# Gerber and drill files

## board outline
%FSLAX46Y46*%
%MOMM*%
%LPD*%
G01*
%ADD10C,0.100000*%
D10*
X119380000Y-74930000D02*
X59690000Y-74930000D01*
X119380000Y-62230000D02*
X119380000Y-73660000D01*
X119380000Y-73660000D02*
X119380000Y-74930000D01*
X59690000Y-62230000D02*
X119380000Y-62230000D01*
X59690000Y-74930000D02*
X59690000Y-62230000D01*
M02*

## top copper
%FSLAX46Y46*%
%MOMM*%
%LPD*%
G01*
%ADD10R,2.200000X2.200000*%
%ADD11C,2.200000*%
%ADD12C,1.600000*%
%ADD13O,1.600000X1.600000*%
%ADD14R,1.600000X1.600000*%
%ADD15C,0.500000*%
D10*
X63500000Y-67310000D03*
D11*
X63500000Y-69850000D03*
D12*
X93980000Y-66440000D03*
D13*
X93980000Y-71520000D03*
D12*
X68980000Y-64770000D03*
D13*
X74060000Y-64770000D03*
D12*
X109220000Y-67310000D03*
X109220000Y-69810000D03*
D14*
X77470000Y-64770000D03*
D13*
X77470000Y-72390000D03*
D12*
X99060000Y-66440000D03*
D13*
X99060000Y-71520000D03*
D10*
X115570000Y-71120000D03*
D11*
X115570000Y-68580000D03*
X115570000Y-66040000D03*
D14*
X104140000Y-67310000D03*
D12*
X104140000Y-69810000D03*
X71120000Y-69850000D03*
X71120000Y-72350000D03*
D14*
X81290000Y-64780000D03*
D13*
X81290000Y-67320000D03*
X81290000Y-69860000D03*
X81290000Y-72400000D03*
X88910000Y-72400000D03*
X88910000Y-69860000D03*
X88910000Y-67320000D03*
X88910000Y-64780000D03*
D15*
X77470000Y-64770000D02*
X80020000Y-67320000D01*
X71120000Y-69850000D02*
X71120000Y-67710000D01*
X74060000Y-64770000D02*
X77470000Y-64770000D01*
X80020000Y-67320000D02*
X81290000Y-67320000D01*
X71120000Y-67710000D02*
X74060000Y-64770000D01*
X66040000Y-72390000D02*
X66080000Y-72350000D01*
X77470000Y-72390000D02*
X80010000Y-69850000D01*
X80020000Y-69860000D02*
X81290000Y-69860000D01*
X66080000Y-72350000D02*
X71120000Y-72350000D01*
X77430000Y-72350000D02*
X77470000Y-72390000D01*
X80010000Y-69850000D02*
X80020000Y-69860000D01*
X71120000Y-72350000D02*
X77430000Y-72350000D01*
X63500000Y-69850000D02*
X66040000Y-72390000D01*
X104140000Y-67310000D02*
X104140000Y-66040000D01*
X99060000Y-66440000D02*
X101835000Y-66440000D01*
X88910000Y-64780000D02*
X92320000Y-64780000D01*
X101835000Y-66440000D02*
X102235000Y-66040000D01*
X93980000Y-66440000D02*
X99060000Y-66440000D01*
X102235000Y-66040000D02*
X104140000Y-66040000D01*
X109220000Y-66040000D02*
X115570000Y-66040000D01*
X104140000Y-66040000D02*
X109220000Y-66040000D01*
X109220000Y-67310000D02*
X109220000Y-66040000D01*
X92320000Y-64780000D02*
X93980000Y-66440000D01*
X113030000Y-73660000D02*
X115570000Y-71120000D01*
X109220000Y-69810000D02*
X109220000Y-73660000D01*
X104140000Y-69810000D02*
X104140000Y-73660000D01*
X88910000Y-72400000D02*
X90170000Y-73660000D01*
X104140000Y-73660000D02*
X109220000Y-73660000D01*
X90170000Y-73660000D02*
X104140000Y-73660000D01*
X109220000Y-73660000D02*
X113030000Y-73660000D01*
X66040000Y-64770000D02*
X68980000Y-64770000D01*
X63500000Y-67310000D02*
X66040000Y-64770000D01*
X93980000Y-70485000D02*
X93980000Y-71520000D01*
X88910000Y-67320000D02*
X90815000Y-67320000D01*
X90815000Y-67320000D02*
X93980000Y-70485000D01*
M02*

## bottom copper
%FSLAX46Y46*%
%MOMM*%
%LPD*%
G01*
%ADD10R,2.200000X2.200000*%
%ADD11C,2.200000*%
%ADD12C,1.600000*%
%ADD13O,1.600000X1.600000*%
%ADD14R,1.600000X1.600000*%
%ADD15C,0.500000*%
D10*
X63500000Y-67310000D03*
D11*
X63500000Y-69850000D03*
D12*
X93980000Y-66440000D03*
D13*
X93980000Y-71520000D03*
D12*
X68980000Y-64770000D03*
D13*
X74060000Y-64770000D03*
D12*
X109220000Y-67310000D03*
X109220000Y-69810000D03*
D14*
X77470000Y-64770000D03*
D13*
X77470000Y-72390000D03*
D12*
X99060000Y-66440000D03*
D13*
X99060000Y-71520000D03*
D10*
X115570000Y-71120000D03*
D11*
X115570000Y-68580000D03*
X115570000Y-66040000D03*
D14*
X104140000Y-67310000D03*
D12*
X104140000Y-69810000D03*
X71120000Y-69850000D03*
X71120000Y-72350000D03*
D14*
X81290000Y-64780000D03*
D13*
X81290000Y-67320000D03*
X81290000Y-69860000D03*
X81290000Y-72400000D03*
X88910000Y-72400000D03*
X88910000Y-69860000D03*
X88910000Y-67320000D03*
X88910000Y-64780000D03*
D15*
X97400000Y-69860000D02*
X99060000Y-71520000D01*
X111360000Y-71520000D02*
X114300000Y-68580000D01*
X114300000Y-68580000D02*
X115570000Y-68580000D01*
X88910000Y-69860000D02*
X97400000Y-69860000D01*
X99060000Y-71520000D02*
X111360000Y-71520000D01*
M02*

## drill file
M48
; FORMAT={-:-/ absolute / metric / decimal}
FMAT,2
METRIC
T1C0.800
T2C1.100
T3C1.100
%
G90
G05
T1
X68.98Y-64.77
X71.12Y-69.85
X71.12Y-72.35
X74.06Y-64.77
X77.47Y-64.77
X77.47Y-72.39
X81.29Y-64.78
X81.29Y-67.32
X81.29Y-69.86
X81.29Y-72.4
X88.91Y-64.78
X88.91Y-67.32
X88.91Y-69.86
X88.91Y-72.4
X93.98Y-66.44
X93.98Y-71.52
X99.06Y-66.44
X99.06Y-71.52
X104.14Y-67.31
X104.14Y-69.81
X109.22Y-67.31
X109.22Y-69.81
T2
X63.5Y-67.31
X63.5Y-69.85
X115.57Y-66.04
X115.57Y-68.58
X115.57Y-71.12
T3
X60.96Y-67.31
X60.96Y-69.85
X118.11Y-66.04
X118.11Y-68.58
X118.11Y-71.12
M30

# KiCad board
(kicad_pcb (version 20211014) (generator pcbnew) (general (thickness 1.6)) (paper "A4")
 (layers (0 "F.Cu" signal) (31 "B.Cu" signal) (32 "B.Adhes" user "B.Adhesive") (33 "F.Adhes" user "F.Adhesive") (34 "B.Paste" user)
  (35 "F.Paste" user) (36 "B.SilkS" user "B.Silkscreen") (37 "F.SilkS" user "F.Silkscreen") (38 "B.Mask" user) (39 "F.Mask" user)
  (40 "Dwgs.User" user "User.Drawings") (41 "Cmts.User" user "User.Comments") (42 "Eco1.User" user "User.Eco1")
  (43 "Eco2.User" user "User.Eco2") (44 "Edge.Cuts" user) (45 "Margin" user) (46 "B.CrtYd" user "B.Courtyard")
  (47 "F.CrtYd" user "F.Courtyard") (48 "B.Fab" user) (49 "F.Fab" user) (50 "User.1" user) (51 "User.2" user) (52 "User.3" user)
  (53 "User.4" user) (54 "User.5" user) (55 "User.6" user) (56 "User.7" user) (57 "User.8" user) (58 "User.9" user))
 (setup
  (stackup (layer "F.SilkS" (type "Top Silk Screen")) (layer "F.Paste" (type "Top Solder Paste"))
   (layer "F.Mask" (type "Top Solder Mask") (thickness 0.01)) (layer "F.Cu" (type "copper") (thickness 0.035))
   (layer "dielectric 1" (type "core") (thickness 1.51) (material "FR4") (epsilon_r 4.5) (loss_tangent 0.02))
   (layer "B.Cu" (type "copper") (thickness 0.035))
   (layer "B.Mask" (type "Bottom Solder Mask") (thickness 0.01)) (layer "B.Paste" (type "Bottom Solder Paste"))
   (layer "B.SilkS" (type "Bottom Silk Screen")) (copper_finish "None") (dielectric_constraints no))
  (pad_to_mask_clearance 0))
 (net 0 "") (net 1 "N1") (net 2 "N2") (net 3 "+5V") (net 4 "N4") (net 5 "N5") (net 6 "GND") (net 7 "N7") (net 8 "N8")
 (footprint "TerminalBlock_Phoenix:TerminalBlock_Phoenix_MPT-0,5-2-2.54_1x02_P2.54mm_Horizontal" (layer "F.Cu") (at 63.5 67.31 -90)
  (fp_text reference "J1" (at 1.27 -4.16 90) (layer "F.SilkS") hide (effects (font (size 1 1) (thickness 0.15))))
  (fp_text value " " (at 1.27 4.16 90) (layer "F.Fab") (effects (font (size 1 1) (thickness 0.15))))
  (pad "" np_thru_hole circle (at 2.54 2.54 270) (size 1.1 1.1) (drill 1.1) (layers *.Cu *.Mask))
  (pad "" np_thru_hole circle (at 0 2.54 270) (size 1.1 1.1) (drill 1.1) (layers *.Cu *.Mask))
  (pad "1" thru_hole rect (at 0 0 270) (size 2.2 2.2) (drill 1.1) (layers *.Cu *.Mask) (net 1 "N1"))
  (pad "2" thru_hole circle (at 2.54 0 270) (size 2.2 2.2) (drill 1.1) (layers *.Cu *.Mask) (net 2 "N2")))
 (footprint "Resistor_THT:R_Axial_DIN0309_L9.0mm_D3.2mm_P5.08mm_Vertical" (layer "F.Cu") (at 93.98 66.44 -90)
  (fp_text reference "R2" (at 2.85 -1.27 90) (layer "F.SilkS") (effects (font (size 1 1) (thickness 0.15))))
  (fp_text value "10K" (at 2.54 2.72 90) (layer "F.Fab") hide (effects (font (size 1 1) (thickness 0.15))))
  (pad "1" thru_hole circle (at 0 0 270) (size 1.6 1.6) (drill 0.8) (layers *.Cu *.Mask) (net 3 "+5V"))
  (pad "2" thru_hole oval (at 5.08 0 270) (size 1.6 1.6) (drill 0.8) (layers *.Cu *.Mask) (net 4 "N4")))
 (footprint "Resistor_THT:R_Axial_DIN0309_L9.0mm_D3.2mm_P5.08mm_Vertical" (layer "F.Cu") (at 68.98 64.77)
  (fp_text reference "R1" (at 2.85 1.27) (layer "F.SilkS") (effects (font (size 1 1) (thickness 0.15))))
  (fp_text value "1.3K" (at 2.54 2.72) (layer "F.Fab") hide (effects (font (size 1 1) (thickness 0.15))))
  (pad "1" thru_hole circle (at 0 0) (size 1.6 1.6) (drill 0.8) (layers *.Cu *.Mask) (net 1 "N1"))
  (pad "2" thru_hole oval (at 5.08 0) (size 1.6 1.6) (drill 0.8) (layers *.Cu *.Mask) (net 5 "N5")))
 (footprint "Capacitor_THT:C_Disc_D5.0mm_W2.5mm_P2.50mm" (layer "F.Cu") (at 109.22 67.31 -90)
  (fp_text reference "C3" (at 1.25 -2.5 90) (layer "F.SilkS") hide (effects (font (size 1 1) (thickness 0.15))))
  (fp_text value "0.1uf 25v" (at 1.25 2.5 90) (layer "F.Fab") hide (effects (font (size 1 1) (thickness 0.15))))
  (pad "1" thru_hole circle (at 0 0 270) (size 1.6 1.6) (drill 0.8) (layers *.Cu *.Mask) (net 3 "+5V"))
  (pad "2" thru_hole circle (at 2.5 0 270) (size 1.6 1.6) (drill 0.8) (layers *.Cu *.Mask) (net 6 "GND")))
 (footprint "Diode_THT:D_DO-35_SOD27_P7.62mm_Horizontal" (layer "F.Cu") (at 77.47 64.77 -90)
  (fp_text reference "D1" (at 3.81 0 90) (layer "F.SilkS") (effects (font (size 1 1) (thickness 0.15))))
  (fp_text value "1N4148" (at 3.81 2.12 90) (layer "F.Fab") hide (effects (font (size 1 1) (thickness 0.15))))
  (pad "1" thru_hole rect (at 0 0 270) (size 1.6 1.6) (drill 0.8) (layers *.Cu *.Mask) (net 5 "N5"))
  (pad "2" thru_hole oval (at 7.62 0 270) (size 1.6 1.6) (drill 0.8) (layers *.Cu *.Mask) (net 2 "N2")))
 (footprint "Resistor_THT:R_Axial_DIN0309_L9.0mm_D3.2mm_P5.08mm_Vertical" (layer "F.Cu") (at 99.06 66.44 -90)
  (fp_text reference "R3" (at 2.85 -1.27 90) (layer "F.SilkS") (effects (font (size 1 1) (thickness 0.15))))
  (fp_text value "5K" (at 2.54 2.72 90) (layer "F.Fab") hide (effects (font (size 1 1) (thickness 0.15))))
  (pad "1" thru_hole circle (at 0 0 270) (size 1.6 1.6) (drill 0.8) (layers *.Cu *.Mask) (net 3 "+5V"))
  (pad "2" thru_hole oval (at 5.08 0 270) (size 1.6 1.6) (drill 0.8) (layers *.Cu *.Mask) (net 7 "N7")))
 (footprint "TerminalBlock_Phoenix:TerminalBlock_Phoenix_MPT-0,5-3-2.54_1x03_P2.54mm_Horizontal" (layer "F.Cu") (at 115.57 71.12 90)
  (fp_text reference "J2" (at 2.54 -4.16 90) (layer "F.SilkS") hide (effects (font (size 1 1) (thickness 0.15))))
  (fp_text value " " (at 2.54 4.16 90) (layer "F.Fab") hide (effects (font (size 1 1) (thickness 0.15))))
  (pad "" np_thru_hole circle (at 2.54 2.54 90) (size 1.1 1.1) (drill 1.1) (layers *.Cu *.Mask))
  (pad "" np_thru_hole circle (at 0 2.54 90) (size 1.1 1.1) (drill 1.1) (layers *.Cu *.Mask))
  (pad "" np_thru_hole circle (at 5.08 2.54 90) (size 1.1 1.1) (drill 1.1) (layers *.Cu *.Mask))
  (pad "1" thru_hole rect (at 0 0 90) (size 2.2 2.2) (drill 1.1) (layers *.Cu *.Mask) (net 6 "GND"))
  (pad "2" thru_hole circle (at 2.54 0 90) (size 2.2 2.2) (drill 1.1) (layers *.Cu *.Mask) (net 7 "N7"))
  (pad "3" thru_hole circle (at 5.08 0 90) (size 2.2 2.2) (drill 1.1) (layers *.Cu *.Mask) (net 3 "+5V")))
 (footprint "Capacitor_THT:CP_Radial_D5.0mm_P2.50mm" (layer "F.Cu") (at 104.14 67.31 -90)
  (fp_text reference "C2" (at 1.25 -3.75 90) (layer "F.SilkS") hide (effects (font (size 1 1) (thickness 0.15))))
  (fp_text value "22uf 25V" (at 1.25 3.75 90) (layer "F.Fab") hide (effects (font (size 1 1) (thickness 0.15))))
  (pad "1" thru_hole rect (at 0 0 270) (size 1.6 1.6) (drill 0.8) (layers *.Cu *.Mask) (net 3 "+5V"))
  (pad "2" thru_hole circle (at 2.5 0 270) (size 1.6 1.6) (drill 0.8) (layers *.Cu *.Mask) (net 6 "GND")))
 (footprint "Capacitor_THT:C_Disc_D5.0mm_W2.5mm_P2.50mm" (layer "F.Cu") (at 71.12 69.85 -90)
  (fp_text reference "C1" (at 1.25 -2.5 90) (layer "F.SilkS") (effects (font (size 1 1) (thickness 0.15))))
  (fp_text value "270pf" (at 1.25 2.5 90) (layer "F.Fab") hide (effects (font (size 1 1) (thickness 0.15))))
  (pad "1" thru_hole circle (at 0 0 270) (size 1.6 1.6) (drill 0.8) (layers *.Cu *.Mask) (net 5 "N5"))
  (pad "2" thru_hole circle (at 2.5 0 270) (size 1.6 1.6) (drill 0.8) (layers *.Cu *.Mask) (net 2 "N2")))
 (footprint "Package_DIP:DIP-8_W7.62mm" (layer "F.Cu") (at 81.29 64.78)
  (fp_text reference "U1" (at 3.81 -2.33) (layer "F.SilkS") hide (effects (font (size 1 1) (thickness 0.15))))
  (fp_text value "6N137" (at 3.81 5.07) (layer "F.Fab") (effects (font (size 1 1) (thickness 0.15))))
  (pad "1" thru_hole rect (at 0 0) (size 1.6 1.6) (drill 0.8) (layers *.Cu *.Mask) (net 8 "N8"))
  (pad "2" thru_hole oval (at 0 2.54) (size 1.6 1.6) (drill 0.8) (layers *.Cu *.Mask) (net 5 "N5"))
  (pad "3" thru_hole oval (at 0 5.08) (size 1.6 1.6) (drill 0.8) (layers *.Cu *.Mask) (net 2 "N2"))
  (pad "4" thru_hole oval (at 0 7.62) (size 1.6 1.6) (drill 0.8) (layers *.Cu *.Mask))
  (pad "5" thru_hole oval (at 7.62 7.62) (size 1.6 1.6) (drill 0.8) (layers *.Cu *.Mask) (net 6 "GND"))
  (pad "6" thru_hole oval (at 7.62 5.08) (size 1.6 1.6) (drill 0.8) (layers *.Cu *.Mask) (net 7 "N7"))
  (pad "7" thru_hole oval (at 7.62 2.54) (size 1.6 1.6) (drill 0.8) (layers *.Cu *.Mask) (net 4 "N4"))
  (pad "8" thru_hole oval (at 7.62 0) (size 1.6 1.6) (drill 0.8) (layers *.Cu *.Mask) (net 3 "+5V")))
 (gr_line (start 119.38 74.93) (end 59.69 74.93) (layer "Edge.Cuts") (width 0.1))
 (gr_line (start 119.38 62.23) (end 119.38 73.66) (layer "Edge.Cuts") (width 0.1))
 (gr_line (start 119.38 73.66) (end 119.38 74.93) (layer "Edge.Cuts") (width 0.1))
 (gr_line (start 59.69 62.23) (end 119.38 62.23) (layer "Edge.Cuts") (width 0.1))
 (gr_line (start 59.69 74.93) (end 59.69 62.23) (layer "Edge.Cuts") (width 0.1))
 (segment (start 77.47 64.77) (end 80.02 67.32) (width 0.5) (layer "F.Cu") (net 5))
 (segment (start 71.12 69.85) (end 71.12 67.71) (width 0.5) (layer "F.Cu") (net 5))
 (segment (start 74.06 64.77) (end 77.47 64.77) (width 0.5) (layer "F.Cu") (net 5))
 (segment (start 80.02 67.32) (end 81.29 67.32) (width 0.5) (layer "F.Cu") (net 5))
 (segment (start 71.12 67.71) (end 74.06 64.77) (width 0.5) (layer "F.Cu") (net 5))
 (segment (start 66.04 72.39) (end 66.08 72.35) (width 0.5) (layer "F.Cu") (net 2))
 (segment (start 77.47 72.39) (end 80.01 69.85) (width 0.5) (layer "F.Cu") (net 2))
 (segment (start 80.02 69.86) (end 81.29 69.86) (width 0.5) (layer "F.Cu") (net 2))
 (segment (start 66.08 72.35) (end 71.12 72.35) (width 0.5) (layer "F.Cu") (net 2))
 (segment (start 77.43 72.35) (end 77.47 72.39) (width 0.5) (layer "F.Cu") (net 2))
 (segment (start 80.01 69.85) (end 80.02 69.86) (width 0.5) (layer "F.Cu") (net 2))
 (segment (start 71.12 72.35) (end 77.43 72.35) (width 0.5) (layer "F.Cu") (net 2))
 (segment (start 63.5 69.85) (end 66.04 72.39) (width 0.5) (layer "F.Cu") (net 2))
 (segment (start 104.14 67.31) (end 104.14 66.04) (width 0.5) (layer "F.Cu") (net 3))
 (segment (start 99.06 66.44) (end 101.835 66.44) (width 0.5) (layer "F.Cu") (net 3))
 (segment (start 88.91 64.78) (end 92.32 64.78) (width 0.5) (layer "F.Cu") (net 3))
 (segment (start 101.835 66.44) (end 102.235 66.04) (width 0.5) (layer "F.Cu") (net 3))
 (segment (start 93.98 66.44) (end 99.06 66.44) (width 0.5) (layer "F.Cu") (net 3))
 (segment (start 102.235 66.04) (end 104.14 66.04) (width 0.5) (layer "F.Cu") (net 3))
 (segment (start 109.22 66.04) (end 115.57 66.04) (width 0.5) (layer "F.Cu") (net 3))
 (segment (start 104.14 66.04) (end 109.22 66.04) (width 0.5) (layer "F.Cu") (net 3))
 (segment (start 109.22 67.31) (end 109.22 66.04) (width 0.5) (layer "F.Cu") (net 3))
 (segment (start 92.32 64.78) (end 93.98 66.44) (width 0.5) (layer "F.Cu") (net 3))
 (segment (start 113.03 73.66) (end 115.57 71.12) (width 0.5) (layer "F.Cu") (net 6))
 (segment (start 109.22 69.81) (end 109.22 73.66) (width 0.5) (layer "F.Cu") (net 6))
 (segment (start 104.14 69.81) (end 104.14 73.66) (width 0.5) (layer "F.Cu") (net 6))
 (segment (start 88.91 72.4) (end 90.17 73.66) (width 0.5) (layer "F.Cu") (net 6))
 (segment (start 104.14 73.66) (end 109.22 73.66) (width 0.5) (layer "F.Cu") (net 6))
 (segment (start 90.17 73.66) (end 104.14 73.66) (width 0.5) (layer "F.Cu") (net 6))
 (segment (start 109.22 73.66) (end 113.03 73.66) (width 0.5) (layer "F.Cu") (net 6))
 (segment (start 66.04 64.77) (end 68.98 64.77) (width 0.5) (layer "F.Cu") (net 1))
 (segment (start 63.5 67.31) (end 66.04 64.77) (width 0.5) (layer "F.Cu") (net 1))
 (segment (start 97.4 69.86) (end 99.06 71.52) (width 0.5) (layer "B.Cu") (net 7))
 (segment (start 111.36 71.52) (end 114.3 68.58) (width 0.5) (layer "B.Cu") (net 7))
 (segment (start 114.3 68.58) (end 115.57 68.58) (width 0.5) (layer "B.Cu") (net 7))
 (segment (start 88.91 69.86) (end 97.4 69.86) (width 0.5) (layer "B.Cu") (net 7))
 (segment (start 99.06 71.52) (end 111.36 71.52) (width 0.5) (layer "B.Cu") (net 7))
 (segment (start 93.98 70.485) (end 93.98 71.52) (width 0.5) (layer "F.Cu") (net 4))
 (segment (start 88.91 67.32) (end 90.815 67.32) (width 0.5) (layer "F.Cu") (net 4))
 (segment (start 90.815 67.32) (end 93.98 70.485) (width 0.5) (layer "F.Cu") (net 4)))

